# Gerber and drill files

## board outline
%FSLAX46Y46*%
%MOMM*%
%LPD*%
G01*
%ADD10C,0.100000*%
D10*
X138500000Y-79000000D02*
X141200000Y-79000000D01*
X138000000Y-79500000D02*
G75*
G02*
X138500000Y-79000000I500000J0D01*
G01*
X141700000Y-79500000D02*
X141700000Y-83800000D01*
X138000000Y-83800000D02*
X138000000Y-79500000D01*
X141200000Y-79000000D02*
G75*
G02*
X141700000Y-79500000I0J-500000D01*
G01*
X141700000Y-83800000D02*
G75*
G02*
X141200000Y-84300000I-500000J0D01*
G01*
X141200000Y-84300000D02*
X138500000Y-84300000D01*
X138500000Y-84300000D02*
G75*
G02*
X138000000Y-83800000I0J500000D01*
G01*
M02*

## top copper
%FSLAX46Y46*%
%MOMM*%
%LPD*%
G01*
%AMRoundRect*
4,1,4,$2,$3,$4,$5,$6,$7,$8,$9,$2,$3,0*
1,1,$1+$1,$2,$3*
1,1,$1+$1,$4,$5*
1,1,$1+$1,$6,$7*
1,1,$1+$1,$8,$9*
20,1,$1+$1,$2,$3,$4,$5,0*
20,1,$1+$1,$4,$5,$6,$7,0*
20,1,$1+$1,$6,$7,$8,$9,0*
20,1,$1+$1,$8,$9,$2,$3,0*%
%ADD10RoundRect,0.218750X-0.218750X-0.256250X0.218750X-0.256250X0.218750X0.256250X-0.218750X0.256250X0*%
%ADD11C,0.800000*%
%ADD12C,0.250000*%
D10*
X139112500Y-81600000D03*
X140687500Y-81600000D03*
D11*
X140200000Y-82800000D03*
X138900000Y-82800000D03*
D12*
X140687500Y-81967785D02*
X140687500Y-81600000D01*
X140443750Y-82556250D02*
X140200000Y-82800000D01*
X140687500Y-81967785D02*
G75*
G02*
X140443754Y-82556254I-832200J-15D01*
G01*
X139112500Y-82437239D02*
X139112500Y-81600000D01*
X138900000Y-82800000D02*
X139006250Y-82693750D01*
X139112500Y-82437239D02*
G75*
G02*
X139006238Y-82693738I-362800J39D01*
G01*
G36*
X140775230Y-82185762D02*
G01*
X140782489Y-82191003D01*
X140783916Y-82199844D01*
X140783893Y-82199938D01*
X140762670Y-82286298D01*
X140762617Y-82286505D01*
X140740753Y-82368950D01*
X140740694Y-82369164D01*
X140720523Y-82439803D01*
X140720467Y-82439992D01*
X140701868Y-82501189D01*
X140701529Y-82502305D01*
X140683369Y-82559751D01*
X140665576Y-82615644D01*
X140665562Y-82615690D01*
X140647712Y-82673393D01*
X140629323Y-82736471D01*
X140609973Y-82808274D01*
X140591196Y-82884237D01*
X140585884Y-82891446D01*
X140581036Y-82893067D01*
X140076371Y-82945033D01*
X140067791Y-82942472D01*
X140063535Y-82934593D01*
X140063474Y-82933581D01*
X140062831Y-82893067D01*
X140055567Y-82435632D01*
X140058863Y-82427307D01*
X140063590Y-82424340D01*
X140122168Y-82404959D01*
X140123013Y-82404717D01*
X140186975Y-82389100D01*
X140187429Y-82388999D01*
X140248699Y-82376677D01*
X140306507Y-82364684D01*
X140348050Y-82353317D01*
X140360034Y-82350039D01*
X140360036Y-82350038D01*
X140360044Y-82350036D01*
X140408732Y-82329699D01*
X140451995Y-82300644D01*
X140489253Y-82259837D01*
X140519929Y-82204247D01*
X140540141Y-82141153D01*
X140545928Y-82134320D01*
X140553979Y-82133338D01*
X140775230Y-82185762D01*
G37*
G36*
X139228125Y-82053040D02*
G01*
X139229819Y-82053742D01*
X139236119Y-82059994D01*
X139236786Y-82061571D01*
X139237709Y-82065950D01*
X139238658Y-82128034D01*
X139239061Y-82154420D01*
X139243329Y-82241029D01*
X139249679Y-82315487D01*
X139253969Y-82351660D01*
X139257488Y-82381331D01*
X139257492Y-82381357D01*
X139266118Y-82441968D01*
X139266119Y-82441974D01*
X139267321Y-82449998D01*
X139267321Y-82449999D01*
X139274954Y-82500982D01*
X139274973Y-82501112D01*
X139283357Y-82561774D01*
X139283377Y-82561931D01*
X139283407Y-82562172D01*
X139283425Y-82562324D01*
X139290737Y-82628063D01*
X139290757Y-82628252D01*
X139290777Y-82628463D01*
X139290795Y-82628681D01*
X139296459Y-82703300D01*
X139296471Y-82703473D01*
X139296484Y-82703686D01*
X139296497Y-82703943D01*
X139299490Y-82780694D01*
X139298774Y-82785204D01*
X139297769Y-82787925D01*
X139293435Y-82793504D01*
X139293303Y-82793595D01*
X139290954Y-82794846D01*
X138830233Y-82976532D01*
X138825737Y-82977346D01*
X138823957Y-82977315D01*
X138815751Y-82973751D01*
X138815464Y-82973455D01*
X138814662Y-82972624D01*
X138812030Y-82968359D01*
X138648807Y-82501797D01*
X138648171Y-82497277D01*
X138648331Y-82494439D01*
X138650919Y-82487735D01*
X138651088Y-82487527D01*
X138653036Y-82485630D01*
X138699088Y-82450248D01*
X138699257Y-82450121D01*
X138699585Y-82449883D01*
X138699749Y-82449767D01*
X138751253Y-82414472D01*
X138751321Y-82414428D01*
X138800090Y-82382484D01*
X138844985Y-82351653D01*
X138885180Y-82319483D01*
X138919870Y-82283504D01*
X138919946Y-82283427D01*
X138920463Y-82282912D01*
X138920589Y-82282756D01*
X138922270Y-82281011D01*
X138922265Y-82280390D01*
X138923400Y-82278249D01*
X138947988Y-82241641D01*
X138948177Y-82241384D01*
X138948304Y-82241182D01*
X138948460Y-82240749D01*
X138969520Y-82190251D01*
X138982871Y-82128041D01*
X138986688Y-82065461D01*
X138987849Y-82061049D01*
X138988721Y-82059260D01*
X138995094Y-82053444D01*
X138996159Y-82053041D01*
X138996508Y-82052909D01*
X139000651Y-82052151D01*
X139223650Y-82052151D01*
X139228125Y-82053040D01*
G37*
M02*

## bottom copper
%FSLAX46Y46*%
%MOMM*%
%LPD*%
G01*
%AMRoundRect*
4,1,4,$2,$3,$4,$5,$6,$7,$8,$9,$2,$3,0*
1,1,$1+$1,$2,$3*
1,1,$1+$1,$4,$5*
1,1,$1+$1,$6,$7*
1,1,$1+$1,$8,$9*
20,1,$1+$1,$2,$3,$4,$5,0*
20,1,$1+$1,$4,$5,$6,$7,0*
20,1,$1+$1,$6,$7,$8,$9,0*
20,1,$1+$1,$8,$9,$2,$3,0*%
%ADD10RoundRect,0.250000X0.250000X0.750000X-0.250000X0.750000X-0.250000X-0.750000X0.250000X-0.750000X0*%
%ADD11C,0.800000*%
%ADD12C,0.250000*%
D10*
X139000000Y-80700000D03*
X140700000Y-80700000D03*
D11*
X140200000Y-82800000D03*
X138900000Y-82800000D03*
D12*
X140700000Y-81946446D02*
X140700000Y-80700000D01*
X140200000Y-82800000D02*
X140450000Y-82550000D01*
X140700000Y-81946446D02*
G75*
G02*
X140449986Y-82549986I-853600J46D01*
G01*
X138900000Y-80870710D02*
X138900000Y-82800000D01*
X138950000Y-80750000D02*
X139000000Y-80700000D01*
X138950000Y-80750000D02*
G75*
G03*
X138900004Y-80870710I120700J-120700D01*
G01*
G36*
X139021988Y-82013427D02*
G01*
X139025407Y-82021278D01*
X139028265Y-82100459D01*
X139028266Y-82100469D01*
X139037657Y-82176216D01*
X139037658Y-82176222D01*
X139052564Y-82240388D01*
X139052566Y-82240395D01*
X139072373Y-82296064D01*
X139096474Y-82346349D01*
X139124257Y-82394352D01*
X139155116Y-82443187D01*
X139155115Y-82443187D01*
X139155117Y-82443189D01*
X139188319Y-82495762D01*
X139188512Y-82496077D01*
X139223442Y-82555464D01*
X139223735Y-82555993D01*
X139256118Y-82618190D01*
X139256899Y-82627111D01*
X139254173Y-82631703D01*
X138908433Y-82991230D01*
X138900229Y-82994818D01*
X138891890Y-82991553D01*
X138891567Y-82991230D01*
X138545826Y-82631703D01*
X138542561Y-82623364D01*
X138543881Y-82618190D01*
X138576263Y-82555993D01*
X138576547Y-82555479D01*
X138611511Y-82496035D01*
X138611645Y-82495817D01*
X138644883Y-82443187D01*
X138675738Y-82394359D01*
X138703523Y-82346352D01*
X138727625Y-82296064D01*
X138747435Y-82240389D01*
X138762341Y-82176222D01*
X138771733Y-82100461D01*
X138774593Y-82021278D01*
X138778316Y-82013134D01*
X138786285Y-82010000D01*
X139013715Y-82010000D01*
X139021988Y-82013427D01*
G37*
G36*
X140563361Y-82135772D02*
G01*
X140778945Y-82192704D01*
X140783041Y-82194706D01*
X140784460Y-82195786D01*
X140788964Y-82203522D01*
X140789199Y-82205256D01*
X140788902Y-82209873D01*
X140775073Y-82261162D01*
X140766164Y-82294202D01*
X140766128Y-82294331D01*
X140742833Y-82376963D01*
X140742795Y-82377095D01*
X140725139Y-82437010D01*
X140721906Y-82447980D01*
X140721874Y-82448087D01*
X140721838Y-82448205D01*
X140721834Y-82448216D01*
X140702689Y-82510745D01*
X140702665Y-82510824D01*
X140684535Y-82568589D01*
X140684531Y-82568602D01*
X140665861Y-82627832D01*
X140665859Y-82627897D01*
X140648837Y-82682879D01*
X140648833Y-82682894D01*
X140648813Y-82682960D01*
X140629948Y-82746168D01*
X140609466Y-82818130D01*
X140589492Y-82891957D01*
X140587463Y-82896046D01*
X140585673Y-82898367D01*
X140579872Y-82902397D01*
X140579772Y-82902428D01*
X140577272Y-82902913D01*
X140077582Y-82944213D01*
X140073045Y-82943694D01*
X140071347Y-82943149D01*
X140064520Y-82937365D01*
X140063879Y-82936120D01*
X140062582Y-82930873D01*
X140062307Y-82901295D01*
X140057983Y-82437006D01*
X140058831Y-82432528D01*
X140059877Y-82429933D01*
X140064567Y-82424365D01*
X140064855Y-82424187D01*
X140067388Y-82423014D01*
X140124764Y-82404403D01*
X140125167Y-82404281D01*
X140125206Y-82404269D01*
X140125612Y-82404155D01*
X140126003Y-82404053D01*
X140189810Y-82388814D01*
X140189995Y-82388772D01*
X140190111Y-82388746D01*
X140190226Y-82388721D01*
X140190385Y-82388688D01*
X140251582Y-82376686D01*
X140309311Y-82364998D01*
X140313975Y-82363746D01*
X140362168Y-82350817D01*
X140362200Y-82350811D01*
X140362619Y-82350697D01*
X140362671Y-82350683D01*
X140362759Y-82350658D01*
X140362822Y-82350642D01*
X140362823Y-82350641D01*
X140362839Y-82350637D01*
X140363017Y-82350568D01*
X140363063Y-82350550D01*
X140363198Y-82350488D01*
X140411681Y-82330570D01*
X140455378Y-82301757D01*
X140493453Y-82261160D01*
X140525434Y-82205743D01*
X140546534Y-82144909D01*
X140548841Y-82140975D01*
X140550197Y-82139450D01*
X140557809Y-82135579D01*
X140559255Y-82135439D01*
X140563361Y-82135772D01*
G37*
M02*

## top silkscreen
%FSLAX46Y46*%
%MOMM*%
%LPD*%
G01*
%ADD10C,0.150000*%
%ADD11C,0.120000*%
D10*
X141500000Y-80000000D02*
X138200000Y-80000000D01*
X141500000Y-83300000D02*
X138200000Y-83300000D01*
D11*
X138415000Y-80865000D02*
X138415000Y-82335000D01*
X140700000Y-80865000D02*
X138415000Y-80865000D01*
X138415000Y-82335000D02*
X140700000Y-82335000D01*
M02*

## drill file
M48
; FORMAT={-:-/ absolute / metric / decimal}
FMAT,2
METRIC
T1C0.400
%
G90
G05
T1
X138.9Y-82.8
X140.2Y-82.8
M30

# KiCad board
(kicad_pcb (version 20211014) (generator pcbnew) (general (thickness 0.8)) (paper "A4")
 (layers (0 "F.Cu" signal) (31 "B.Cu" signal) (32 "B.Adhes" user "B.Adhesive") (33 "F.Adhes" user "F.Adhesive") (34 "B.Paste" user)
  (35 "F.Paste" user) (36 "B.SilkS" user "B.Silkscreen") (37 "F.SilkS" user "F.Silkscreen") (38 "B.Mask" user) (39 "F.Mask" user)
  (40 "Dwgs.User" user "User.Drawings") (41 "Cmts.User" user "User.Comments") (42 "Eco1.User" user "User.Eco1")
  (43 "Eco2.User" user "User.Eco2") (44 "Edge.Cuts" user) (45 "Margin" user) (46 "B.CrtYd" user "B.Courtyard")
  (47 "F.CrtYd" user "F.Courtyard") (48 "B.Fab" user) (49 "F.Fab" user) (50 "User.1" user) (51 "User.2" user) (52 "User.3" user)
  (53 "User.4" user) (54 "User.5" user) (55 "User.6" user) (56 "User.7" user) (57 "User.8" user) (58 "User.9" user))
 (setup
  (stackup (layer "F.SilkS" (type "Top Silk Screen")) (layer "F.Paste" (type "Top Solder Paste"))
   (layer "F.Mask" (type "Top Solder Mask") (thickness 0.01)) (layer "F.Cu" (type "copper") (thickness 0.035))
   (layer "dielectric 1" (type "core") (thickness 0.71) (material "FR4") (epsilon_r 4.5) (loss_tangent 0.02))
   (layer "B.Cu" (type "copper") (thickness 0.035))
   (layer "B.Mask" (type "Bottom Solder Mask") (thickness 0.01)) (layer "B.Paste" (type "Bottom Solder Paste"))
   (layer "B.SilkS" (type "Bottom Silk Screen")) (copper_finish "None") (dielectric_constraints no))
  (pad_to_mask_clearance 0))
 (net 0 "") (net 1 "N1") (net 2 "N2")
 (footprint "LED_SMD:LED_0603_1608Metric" (layer "F.Cu") (at 139.9 81.6)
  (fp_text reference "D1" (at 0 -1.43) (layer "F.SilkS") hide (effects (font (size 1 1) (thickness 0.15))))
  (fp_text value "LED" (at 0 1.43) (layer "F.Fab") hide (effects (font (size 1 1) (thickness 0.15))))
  (fp_line (start -1.485 -0.735) (end -1.485 0.735) (layer "F.SilkS") (width 0.12))
  (fp_line (start 0.8 -0.735) (end -1.485 -0.735) (layer "F.SilkS") (width 0.12))
  (fp_line (start -1.485 0.735) (end 0.8 0.735) (layer "F.SilkS") (width 0.12))
  (pad "1" smd roundrect (at -0.7875 0) (size 0.875 0.95) (layers "F.Cu" "F.Paste" "F.Mask") (roundrect_rratio 0.25) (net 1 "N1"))
  (pad "2" smd roundrect (at 0.7875 0) (size 0.875 0.95) (layers "F.Cu" "F.Paste" "F.Mask") (roundrect_rratio 0.25) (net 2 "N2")))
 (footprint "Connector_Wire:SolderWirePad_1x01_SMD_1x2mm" (layer "B.Cu") (at 139 80.7 180)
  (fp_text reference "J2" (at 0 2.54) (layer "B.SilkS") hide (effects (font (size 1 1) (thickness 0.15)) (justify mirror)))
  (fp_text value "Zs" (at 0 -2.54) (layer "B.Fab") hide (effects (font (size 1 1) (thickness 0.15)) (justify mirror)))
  (pad "1" smd roundrect (at 0 0 180) (size 1 2) (layers "B.Cu" "B.Paste" "B.Mask") (roundrect_rratio 0.25) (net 1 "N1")))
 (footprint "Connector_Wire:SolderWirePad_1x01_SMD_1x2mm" (layer "B.Cu") (at 140.7 80.7 180)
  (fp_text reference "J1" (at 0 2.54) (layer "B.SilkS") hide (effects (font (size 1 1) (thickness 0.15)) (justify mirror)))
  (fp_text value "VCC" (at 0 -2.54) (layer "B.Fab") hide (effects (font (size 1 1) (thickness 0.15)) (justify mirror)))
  (pad "1" smd roundrect (at 0 0 180) (size 1 2) (layers "B.Cu" "B.Paste" "B.Mask") (roundrect_rratio 0.25) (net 2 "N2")))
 (gr_line (start 141.5 80) (end 138.2 80) (layer "F.SilkS") (width 0.15))
 (gr_line (start 141.5 83.3) (end 138.2 83.3) (layer "F.SilkS") (width 0.15))
 (gr_line (start 138.5 79) (end 141.2 79) (layer "Edge.Cuts") (width 0.1))
 (gr_arc (start 138 79.5) (mid 138.146447 79.146447) (end 138.5 79) (layer "Edge.Cuts") (width 0.1))
 (gr_line (start 141.7 79.5) (end 141.7 83.8) (layer "Edge.Cuts") (width 0.1))
 (gr_line (start 138 83.8) (end 138 79.5) (layer "Edge.Cuts") (width 0.1))
 (gr_arc (start 141.2 79) (mid 141.553553 79.146447) (end 141.7 79.5) (layer "Edge.Cuts") (width 0.1))
 (gr_arc (start 141.7 83.8) (mid 141.553553 84.153553) (end 141.2 84.3) (layer "Edge.Cuts") (width 0.1))
 (gr_line (start 141.2 84.3) (end 138.5 84.3) (layer "Edge.Cuts") (width 0.1))
 (gr_arc (start 138.5 84.3) (mid 138.146447 84.153553) (end 138 83.8) (layer "Edge.Cuts") (width 0.1))
 (segment (start 140.6875 81.967785) (end 140.6875 81.6) (width 0.25) (layer "F.Cu") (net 2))
 (segment (start 140.44375 82.55625) (end 140.2 82.8) (width 0.25) (layer "F.Cu") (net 2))
 (via (at 140.2 82.8) (size 0.8) (drill 0.4) (layers "F.Cu" "B.Cu") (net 2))
 (arc (start 140.6875 81.967785) (mid 140.624151 82.28626) (end 140.44375 82.55625) (width 0.25) (layer "F.Cu") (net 2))
 (segment (start 140.7 81.946446) (end 140.7 80.7) (width 0.25) (layer "B.Cu") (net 2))
 (segment (start 140.2 82.8) (end 140.45 82.55) (width 0.25) (layer "B.Cu") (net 2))
 (arc (start 140.7 81.946446) (mid 140.635027 82.273087) (end 140.45 82.55) (width 0.25) (layer "B.Cu") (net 2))
 (segment (start 139.1125 82.437239) (end 139.1125 81.6) (width 0.25) (layer "F.Cu") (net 1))
 (segment (start 138.9 82.8) (end 139.00625 82.69375) (width 0.25) (layer "F.Cu") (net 1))
 (via (at 138.9 82.8) (size 0.8) (drill 0.4) (layers "F.Cu" "B.Cu") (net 1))
 (arc (start 139.1125 82.437239) (mid 139.084886 82.576061) (end 139.00625 82.69375) (width 0.25) (layer "F.Cu") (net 1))
 (segment (start 138.9 80.87071) (end 138.9 82.8) (width 0.25) (layer "B.Cu") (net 1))
 (segment (start 138.95 80.75) (end 139 80.7) (width 0.25) (layer "B.Cu") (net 1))
 (arc (start 138.95 80.75) (mid 138.912994 80.805382) (end 138.9 80.87071) (width 0.25) (layer "B.Cu") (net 1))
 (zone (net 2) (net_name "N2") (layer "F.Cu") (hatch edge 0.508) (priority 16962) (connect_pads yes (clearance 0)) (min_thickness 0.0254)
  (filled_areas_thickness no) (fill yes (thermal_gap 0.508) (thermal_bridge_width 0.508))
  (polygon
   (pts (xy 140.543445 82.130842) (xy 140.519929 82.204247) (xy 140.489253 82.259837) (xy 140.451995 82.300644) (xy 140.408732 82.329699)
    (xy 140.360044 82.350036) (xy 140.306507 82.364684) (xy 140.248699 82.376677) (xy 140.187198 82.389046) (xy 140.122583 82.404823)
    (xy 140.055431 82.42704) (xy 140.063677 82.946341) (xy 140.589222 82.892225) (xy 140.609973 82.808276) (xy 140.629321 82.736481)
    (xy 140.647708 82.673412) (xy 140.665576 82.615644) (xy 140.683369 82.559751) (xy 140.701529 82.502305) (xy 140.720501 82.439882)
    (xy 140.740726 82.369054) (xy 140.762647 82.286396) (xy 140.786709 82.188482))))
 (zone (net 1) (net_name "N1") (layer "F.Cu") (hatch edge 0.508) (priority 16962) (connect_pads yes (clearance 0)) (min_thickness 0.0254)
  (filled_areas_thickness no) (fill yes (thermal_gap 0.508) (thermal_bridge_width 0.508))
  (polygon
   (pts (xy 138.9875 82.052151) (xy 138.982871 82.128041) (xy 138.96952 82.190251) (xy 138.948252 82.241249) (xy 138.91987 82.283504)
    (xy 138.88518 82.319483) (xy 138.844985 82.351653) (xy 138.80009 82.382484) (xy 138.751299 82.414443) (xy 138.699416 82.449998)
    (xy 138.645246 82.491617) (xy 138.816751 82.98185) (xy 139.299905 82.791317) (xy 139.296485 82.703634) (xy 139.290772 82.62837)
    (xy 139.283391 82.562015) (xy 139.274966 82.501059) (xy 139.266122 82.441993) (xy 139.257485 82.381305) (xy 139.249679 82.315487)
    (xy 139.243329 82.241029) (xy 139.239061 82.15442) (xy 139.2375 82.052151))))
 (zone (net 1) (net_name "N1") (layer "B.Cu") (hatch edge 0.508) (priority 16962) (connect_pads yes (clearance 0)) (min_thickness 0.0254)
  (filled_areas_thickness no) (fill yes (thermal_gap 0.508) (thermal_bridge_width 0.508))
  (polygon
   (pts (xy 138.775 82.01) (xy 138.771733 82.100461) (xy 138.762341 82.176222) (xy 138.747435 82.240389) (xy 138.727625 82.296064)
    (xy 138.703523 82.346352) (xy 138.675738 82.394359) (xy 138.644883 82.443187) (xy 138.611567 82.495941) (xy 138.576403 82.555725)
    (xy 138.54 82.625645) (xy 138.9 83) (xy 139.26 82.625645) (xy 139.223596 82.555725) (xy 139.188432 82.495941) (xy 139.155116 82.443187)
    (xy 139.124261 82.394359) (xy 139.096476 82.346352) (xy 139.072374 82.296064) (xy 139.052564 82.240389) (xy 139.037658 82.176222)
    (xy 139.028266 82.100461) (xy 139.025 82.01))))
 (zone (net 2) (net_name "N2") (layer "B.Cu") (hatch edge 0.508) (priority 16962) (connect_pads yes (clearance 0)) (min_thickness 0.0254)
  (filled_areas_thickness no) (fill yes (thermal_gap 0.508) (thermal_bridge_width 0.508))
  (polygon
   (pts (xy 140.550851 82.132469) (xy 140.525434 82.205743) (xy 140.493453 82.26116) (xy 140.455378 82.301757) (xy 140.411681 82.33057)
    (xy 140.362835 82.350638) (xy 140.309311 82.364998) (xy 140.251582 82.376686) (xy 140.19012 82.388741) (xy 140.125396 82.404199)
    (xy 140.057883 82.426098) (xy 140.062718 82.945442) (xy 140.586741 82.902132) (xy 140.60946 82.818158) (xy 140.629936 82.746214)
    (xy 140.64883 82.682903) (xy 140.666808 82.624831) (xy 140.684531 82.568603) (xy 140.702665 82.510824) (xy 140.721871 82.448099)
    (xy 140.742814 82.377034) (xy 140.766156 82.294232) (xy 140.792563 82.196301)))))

